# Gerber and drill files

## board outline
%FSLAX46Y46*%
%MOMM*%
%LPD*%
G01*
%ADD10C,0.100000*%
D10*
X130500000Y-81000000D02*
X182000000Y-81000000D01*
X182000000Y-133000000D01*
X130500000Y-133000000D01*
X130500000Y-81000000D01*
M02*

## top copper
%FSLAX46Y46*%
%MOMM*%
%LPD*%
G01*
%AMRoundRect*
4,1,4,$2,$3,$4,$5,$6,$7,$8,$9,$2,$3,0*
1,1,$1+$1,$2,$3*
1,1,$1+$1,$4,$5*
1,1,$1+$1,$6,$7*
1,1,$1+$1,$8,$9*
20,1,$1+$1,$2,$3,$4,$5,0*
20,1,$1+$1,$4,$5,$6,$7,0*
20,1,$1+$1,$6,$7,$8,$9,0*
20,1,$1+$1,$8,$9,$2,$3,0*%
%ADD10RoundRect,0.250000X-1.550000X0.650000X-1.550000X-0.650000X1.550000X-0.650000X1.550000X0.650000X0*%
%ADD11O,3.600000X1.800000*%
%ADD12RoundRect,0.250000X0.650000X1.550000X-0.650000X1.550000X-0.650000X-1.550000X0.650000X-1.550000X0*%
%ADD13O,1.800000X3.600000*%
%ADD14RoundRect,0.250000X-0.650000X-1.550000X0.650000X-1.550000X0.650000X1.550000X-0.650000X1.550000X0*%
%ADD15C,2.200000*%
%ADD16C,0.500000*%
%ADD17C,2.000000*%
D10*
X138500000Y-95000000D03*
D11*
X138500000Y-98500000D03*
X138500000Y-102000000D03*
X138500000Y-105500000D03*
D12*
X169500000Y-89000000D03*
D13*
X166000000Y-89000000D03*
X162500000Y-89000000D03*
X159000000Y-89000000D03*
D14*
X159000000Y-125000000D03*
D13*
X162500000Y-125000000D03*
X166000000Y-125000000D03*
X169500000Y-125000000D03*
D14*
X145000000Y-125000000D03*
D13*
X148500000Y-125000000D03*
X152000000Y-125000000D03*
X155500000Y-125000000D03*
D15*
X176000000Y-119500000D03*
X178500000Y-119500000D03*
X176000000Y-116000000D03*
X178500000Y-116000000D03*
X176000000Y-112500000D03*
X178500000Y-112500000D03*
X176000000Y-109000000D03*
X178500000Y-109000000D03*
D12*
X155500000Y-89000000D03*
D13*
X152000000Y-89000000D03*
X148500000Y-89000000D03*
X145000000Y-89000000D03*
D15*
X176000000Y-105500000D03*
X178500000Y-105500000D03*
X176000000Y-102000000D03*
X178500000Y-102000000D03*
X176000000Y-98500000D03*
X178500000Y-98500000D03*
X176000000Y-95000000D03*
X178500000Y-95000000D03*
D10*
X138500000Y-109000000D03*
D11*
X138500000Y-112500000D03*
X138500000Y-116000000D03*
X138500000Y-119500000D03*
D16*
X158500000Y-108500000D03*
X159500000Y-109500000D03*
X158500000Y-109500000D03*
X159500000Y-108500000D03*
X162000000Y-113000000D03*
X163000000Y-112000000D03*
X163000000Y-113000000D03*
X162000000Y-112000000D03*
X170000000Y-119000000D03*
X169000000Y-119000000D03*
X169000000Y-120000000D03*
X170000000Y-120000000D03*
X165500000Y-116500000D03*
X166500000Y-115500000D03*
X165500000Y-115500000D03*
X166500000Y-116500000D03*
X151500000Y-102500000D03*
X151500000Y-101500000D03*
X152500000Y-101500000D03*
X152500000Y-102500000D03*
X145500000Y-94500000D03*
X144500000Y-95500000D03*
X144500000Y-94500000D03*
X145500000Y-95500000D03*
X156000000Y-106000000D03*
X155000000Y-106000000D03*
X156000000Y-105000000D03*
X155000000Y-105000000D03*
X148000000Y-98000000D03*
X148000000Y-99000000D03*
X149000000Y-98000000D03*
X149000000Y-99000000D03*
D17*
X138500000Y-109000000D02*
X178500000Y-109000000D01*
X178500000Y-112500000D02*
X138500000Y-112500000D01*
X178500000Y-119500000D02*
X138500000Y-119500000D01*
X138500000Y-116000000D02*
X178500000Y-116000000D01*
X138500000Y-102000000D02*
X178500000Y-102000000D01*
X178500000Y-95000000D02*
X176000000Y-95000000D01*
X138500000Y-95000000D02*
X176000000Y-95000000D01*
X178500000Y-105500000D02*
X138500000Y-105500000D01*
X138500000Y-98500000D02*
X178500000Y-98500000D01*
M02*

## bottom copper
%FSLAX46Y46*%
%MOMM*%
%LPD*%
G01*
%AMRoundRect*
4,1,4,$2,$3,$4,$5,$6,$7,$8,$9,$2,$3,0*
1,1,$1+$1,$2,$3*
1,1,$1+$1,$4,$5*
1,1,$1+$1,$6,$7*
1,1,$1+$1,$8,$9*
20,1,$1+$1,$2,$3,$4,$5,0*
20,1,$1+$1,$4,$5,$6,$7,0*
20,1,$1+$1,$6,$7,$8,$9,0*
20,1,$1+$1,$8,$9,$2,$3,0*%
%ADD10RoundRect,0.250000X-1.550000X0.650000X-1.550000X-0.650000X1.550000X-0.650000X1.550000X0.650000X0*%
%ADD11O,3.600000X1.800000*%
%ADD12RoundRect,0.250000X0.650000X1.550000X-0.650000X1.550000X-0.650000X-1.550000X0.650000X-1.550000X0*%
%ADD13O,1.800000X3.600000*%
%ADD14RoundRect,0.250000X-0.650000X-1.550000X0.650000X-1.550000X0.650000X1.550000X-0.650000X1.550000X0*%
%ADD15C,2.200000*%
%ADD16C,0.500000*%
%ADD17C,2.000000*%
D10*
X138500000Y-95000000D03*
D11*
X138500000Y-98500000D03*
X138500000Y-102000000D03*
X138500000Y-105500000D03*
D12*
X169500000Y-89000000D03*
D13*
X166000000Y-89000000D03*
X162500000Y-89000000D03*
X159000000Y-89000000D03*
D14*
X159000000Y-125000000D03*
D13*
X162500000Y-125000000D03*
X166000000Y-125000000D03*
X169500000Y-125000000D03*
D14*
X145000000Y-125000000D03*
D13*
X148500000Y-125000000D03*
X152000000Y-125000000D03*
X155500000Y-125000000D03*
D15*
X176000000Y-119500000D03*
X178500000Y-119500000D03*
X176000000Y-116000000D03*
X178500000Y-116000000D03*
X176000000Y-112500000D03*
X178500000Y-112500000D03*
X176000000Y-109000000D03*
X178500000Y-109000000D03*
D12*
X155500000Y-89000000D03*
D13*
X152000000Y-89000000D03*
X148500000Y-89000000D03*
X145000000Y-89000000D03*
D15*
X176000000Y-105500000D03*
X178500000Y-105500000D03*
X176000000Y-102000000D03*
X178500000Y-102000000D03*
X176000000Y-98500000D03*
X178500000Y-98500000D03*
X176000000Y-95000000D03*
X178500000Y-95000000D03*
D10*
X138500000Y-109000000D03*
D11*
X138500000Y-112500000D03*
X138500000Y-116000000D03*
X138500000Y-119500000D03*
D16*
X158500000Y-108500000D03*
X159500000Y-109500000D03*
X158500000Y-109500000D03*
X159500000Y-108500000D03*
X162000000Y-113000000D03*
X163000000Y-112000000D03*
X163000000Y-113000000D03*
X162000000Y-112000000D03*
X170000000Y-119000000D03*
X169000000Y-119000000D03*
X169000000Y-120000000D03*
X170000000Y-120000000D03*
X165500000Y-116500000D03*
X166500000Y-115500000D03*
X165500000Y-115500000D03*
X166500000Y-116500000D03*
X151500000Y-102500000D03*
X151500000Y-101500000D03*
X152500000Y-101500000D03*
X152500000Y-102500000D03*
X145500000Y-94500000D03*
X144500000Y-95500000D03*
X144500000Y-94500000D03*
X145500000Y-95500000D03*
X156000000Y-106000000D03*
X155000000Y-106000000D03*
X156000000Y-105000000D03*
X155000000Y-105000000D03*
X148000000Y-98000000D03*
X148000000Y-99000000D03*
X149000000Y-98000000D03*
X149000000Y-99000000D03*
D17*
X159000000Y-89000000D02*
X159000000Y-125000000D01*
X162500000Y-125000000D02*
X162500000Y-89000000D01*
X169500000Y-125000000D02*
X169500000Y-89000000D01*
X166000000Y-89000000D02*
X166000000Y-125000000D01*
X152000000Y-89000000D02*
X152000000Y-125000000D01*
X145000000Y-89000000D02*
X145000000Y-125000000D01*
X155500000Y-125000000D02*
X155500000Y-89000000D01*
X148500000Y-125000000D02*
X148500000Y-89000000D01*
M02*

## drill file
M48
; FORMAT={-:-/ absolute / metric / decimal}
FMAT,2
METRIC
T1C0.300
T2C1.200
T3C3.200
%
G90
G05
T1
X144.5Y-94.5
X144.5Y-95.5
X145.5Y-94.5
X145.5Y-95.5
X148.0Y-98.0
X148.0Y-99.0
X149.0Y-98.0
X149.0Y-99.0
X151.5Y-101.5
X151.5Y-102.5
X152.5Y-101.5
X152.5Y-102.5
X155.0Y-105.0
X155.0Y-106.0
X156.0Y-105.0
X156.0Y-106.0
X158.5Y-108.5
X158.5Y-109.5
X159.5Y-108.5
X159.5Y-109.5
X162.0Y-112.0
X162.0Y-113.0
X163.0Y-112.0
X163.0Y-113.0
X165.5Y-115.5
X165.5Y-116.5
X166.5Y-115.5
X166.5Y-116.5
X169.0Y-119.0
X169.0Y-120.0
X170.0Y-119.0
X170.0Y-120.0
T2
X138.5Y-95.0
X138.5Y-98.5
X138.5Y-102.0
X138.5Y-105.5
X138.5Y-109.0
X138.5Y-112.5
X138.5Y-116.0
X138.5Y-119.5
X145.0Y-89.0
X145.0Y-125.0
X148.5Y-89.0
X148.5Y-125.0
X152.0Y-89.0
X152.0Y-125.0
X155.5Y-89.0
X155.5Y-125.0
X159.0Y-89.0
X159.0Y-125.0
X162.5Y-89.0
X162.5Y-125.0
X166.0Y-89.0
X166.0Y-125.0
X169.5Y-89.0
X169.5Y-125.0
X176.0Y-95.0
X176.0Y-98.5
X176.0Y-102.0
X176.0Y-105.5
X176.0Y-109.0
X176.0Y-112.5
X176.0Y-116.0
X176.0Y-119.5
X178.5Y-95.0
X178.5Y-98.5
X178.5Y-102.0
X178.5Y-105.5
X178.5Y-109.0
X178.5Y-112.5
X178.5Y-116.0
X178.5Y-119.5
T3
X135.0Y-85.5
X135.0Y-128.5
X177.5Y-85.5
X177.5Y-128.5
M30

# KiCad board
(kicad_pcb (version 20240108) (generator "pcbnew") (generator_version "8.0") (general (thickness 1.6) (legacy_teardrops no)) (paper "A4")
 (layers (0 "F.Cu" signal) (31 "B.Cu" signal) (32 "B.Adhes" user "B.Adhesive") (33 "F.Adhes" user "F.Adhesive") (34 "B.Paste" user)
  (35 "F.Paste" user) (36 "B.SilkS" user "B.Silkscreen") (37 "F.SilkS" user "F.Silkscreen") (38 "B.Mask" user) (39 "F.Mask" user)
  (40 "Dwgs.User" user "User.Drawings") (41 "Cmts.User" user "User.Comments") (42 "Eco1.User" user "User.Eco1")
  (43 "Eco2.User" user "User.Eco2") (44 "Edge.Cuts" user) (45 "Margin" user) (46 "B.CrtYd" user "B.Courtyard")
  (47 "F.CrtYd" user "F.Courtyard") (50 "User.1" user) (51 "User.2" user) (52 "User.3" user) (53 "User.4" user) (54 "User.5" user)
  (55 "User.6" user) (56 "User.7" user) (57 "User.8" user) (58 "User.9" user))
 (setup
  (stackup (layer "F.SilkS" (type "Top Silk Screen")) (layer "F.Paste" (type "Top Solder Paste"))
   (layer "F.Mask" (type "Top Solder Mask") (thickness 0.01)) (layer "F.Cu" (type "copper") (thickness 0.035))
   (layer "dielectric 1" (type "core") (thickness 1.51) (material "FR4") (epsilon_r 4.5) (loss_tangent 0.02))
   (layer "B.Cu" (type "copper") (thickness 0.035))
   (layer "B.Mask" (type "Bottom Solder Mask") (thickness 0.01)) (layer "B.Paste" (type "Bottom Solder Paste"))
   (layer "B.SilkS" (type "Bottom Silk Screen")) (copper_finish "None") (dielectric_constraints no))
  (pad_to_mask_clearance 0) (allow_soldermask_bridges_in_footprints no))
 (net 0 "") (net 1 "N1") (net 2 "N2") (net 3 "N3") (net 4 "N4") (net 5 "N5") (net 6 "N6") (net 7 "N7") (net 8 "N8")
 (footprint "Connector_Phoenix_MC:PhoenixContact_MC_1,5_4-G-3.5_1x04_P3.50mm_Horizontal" (layer "F.Cu") (at 138.5 95 -90)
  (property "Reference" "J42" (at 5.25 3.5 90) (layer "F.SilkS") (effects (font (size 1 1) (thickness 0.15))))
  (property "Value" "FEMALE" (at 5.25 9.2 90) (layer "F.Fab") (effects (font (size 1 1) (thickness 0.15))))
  (pad "1" thru_hole roundrect (at 0 0 270) (size 1.8 3.6) (drill 1.2) (layers "*.Cu" "*.Mask") (remove_unused_layers no)
   (roundrect_rratio 0.138889) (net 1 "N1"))
  (pad "2" thru_hole oval (at 3.5 0 270) (size 1.8 3.6) (drill 1.2) (layers "*.Cu" "*.Mask") (remove_unused_layers no) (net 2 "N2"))
  (pad "3" thru_hole oval (at 7 0 270) (size 1.8 3.6) (drill 1.2) (layers "*.Cu" "*.Mask") (remove_unused_layers no) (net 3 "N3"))
  (pad "4" thru_hole oval (at 10.5 0 270) (size 1.8 3.6) (drill 1.2) (layers "*.Cu" "*.Mask") (remove_unused_layers no) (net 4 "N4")))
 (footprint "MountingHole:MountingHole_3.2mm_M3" (layer "F.Cu") (at 135 128.5)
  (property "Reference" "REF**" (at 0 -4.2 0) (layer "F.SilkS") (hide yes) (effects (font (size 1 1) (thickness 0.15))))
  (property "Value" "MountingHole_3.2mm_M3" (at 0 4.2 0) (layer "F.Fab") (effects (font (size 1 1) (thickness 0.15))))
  (pad "" np_thru_hole circle (at 0 0) (size 3.2 3.2) (drill 3.2) (layers "F&B.Cu" "*.Mask")))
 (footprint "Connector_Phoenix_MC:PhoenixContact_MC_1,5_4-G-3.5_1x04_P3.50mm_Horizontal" (layer "F.Cu") (at 169.5 89 180)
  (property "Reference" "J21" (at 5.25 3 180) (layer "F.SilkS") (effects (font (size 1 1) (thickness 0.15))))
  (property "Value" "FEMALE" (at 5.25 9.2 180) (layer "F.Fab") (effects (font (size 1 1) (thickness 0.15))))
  (pad "1" thru_hole roundrect (at 0 0 180) (size 1.8 3.6) (drill 1.2) (layers "*.Cu" "*.Mask") (remove_unused_layers no)
   (roundrect_rratio 0.138889) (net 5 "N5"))
  (pad "2" thru_hole oval (at 3.5 0 180) (size 1.8 3.6) (drill 1.2) (layers "*.Cu" "*.Mask") (remove_unused_layers no) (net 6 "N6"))
  (pad "3" thru_hole oval (at 7 0 180) (size 1.8 3.6) (drill 1.2) (layers "*.Cu" "*.Mask") (remove_unused_layers no) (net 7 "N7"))
  (pad "4" thru_hole oval (at 10.5 0 180) (size 1.8 3.6) (drill 1.2) (layers "*.Cu" "*.Mask") (remove_unused_layers no) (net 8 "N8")))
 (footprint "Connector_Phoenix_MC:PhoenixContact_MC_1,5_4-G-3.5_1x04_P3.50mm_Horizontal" (layer "F.Cu") (at 159 125)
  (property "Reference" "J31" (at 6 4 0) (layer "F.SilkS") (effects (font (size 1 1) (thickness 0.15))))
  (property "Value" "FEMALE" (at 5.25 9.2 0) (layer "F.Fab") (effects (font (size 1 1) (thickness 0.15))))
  (pad "1" thru_hole roundrect (at 0 0) (size 1.8 3.6) (drill 1.2) (layers "*.Cu" "*.Mask") (remove_unused_layers no)
   (roundrect_rratio 0.138889) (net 8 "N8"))
  (pad "2" thru_hole oval (at 3.5 0) (size 1.8 3.6) (drill 1.2) (layers "*.Cu" "*.Mask") (remove_unused_layers no) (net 7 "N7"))
  (pad "3" thru_hole oval (at 7 0) (size 1.8 3.6) (drill 1.2) (layers "*.Cu" "*.Mask") (remove_unused_layers no) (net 6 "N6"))
  (pad "4" thru_hole oval (at 10.5 0) (size 1.8 3.6) (drill 1.2) (layers "*.Cu" "*.Mask") (remove_unused_layers no) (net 5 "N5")))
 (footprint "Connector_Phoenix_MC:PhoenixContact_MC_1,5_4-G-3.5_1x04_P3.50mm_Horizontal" (layer "F.Cu") (at 145 125)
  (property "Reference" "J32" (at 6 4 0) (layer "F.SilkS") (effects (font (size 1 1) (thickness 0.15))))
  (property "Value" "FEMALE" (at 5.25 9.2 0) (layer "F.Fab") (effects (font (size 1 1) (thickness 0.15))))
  (pad "1" thru_hole roundrect (at 0 0) (size 1.8 3.6) (drill 1.2) (layers "*.Cu" "*.Mask") (remove_unused_layers no)
   (roundrect_rratio 0.138889) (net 1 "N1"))
  (pad "2" thru_hole oval (at 3.5 0) (size 1.8 3.6) (drill 1.2) (layers "*.Cu" "*.Mask") (remove_unused_layers no) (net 2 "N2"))
  (pad "3" thru_hole oval (at 7 0) (size 1.8 3.6) (drill 1.2) (layers "*.Cu" "*.Mask") (remove_unused_layers no) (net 3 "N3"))
  (pad "4" thru_hole oval (at 10.5 0) (size 1.8 3.6) (drill 1.2) (layers "*.Cu" "*.Mask") (remove_unused_layers no) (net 4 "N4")))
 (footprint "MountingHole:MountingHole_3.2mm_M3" (layer "F.Cu") (at 177.5 85.5)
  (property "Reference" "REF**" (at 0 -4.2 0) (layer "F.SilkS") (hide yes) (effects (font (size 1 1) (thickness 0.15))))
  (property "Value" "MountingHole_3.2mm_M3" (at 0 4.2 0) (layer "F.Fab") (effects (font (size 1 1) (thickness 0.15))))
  (pad "" np_thru_hole circle (at 0 0) (size 3.2 3.2) (drill 3.2) (layers "F&B.Cu" "*.Mask")))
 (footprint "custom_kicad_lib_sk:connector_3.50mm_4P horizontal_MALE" (layer "F.Cu") (at 176 114.25 90)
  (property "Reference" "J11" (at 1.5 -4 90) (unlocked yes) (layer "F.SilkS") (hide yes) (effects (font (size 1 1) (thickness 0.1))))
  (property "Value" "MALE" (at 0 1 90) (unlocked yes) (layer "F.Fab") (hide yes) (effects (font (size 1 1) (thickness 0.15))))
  (pad "1" thru_hole circle (at -5.25 0 90) (size 2.2 2.2) (drill 1.2) (layers "*.Cu" "*.Mask") (remove_unused_layers no) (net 5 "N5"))
  (pad "1" thru_hole circle (at -5.25 2.5 90) (size 2.2 2.2) (drill 1.2) (layers "*.Cu" "*.Mask") (remove_unused_layers no) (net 5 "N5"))
  (pad "2" thru_hole circle (at -1.75 0 90) (size 2.2 2.2) (drill 1.2) (layers "*.Cu" "*.Mask") (remove_unused_layers no) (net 6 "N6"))
  (pad "2" thru_hole circle (at -1.75 2.5 90) (size 2.2 2.2) (drill 1.2) (layers "*.Cu" "*.Mask") (remove_unused_layers no) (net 6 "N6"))
  (pad "3" thru_hole circle (at 1.75 0 90) (size 2.2 2.2) (drill 1.2) (layers "*.Cu" "*.Mask") (remove_unused_layers no) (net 7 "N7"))
  (pad "3" thru_hole circle (at 1.75 2.5 90) (size 2.2 2.2) (drill 1.2) (layers "*.Cu" "*.Mask") (remove_unused_layers no) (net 7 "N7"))
  (pad "4" thru_hole circle (at 5.25 0 90) (size 2.2 2.2) (drill 1.2) (layers "*.Cu" "*.Mask") (remove_unused_layers no) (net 8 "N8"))
  (pad "4" thru_hole circle (at 5.25 2.5 90) (size 2.2 2.2) (drill 1.2) (layers "*.Cu" "*.Mask") (remove_unused_layers no) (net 8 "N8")))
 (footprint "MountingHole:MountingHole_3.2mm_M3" (layer "F.Cu") (at 135 85.5)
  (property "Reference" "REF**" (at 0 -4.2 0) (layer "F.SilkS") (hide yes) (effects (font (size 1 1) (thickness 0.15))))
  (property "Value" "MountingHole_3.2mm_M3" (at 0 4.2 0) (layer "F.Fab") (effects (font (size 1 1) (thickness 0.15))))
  (pad "" np_thru_hole circle (at 0 0) (size 3.2 3.2) (drill 3.2) (layers "F&B.Cu" "*.Mask")))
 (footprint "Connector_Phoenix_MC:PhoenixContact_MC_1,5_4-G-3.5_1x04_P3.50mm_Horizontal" (layer "F.Cu") (at 155.5 89 180)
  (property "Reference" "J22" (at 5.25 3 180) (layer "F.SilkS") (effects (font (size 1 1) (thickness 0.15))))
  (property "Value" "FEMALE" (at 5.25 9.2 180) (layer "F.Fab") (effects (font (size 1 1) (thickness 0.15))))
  (pad "1" thru_hole roundrect (at 0 0 180) (size 1.8 3.6) (drill 1.2) (layers "*.Cu" "*.Mask") (remove_unused_layers no)
   (roundrect_rratio 0.138889) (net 4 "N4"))
  (pad "2" thru_hole oval (at 3.5 0 180) (size 1.8 3.6) (drill 1.2) (layers "*.Cu" "*.Mask") (remove_unused_layers no) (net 3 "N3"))
  (pad "3" thru_hole oval (at 7 0 180) (size 1.8 3.6) (drill 1.2) (layers "*.Cu" "*.Mask") (remove_unused_layers no) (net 2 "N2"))
  (pad "4" thru_hole oval (at 10.5 0 180) (size 1.8 3.6) (drill 1.2) (layers "*.Cu" "*.Mask") (remove_unused_layers no) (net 1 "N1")))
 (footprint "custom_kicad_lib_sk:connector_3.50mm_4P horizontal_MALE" (layer "F.Cu") (at 176 100.25 90)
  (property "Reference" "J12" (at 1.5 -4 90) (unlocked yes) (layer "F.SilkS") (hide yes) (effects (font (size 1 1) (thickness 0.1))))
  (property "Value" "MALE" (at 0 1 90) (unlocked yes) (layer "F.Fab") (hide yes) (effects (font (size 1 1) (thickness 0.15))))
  (pad "1" thru_hole circle (at -5.25 0 90) (size 2.2 2.2) (drill 1.2) (layers "*.Cu" "*.Mask") (remove_unused_layers no) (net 4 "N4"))
  (pad "1" thru_hole circle (at -5.25 2.5 90) (size 2.2 2.2) (drill 1.2) (layers "*.Cu" "*.Mask") (remove_unused_layers no) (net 4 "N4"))
  (pad "2" thru_hole circle (at -1.75 0 90) (size 2.2 2.2) (drill 1.2) (layers "*.Cu" "*.Mask") (remove_unused_layers no) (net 3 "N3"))
  (pad "2" thru_hole circle (at -1.75 2.5 90) (size 2.2 2.2) (drill 1.2) (layers "*.Cu" "*.Mask") (remove_unused_layers no) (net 3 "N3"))
  (pad "3" thru_hole circle (at 1.75 0 90) (size 2.2 2.2) (drill 1.2) (layers "*.Cu" "*.Mask") (remove_unused_layers no) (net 2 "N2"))
  (pad "3" thru_hole circle (at 1.75 2.5 90) (size 2.2 2.2) (drill 1.2) (layers "*.Cu" "*.Mask") (remove_unused_layers no) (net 2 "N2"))
  (pad "4" thru_hole circle (at 5.25 0 90) (size 2.2 2.2) (drill 1.2) (layers "*.Cu" "*.Mask") (remove_unused_layers no) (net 1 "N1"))
  (pad "4" thru_hole circle (at 5.25 2.5 90) (size 2.2 2.2) (drill 1.2) (layers "*.Cu" "*.Mask") (remove_unused_layers no) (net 1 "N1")))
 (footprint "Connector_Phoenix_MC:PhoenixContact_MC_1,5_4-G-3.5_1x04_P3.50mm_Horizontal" (layer "F.Cu") (at 138.5 109 -90)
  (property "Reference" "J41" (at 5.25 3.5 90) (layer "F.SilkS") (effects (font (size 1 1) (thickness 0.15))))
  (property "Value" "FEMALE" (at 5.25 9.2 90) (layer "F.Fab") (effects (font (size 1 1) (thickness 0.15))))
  (pad "1" thru_hole roundrect (at 0 0 270) (size 1.8 3.6) (drill 1.2) (layers "*.Cu" "*.Mask") (remove_unused_layers no)
   (roundrect_rratio 0.138889) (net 8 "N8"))
  (pad "2" thru_hole oval (at 3.5 0 270) (size 1.8 3.6) (drill 1.2) (layers "*.Cu" "*.Mask") (remove_unused_layers no) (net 7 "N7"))
  (pad "3" thru_hole oval (at 7 0 270) (size 1.8 3.6) (drill 1.2) (layers "*.Cu" "*.Mask") (remove_unused_layers no) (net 6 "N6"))
  (pad "4" thru_hole oval (at 10.5 0 270) (size 1.8 3.6) (drill 1.2) (layers "*.Cu" "*.Mask") (remove_unused_layers no) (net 5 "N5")))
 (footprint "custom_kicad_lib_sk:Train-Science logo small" (layer "F.Cu") (at 157.226 107.315 90)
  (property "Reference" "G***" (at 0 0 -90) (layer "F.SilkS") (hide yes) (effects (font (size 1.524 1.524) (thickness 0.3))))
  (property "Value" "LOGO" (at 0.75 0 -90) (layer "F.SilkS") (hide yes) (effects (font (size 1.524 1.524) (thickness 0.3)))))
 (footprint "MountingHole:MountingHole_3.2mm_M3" (layer "F.Cu") (at 177.5 128.5)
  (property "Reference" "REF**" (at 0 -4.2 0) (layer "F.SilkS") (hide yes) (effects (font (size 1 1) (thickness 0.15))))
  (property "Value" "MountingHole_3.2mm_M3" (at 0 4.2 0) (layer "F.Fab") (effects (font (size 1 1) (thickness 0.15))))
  (pad "" np_thru_hole circle (at 0 0) (size 3.2 3.2) (drill 3.2) (layers "*.Cu" "*.Mask")))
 (gr_rect (start 130.5 81) (end 182 133) (stroke (width 0.1) (type default)) (fill none) (layer "Edge.Cuts"))
 (segment (start 138.5 109) (end 178.5 109) (width 2) (layer "F.Cu") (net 8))
 (via (at 158.5 108.5) (size 0.5) (drill 0.3) (layers "F.Cu" "B.Cu") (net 8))
 (via (at 159.5 109.5) (size 0.5) (drill 0.3) (layers "F.Cu" "B.Cu") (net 8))
 (via (at 158.5 109.5) (size 0.5) (drill 0.3) (layers "F.Cu" "B.Cu") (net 8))
 (via (at 159.5 108.5) (size 0.5) (drill 0.3) (layers "F.Cu" "B.Cu") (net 8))
 (segment (start 159 89) (end 159 125) (width 2) (layer "B.Cu") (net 8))
 (segment (start 178.5 112.5) (end 138.5 112.5) (width 2) (layer "F.Cu") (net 7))
 (via (at 162 113) (size 0.5) (drill 0.3) (layers "F.Cu" "B.Cu") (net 7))
 (via (at 163 112) (size 0.5) (drill 0.3) (layers "F.Cu" "B.Cu") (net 7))
 (via (at 163 113) (size 0.5) (drill 0.3) (layers "F.Cu" "B.Cu") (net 7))
 (via (at 162 112) (size 0.5) (drill 0.3) (layers "F.Cu" "B.Cu") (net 7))
 (segment (start 162.5 125) (end 162.5 89) (width 2) (layer "B.Cu") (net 7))
 (segment (start 178.5 119.5) (end 138.5 119.5) (width 2) (layer "F.Cu") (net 5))
 (via (at 170 119) (size 0.5) (drill 0.3) (layers "F.Cu" "B.Cu") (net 5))
 (via (at 169 119) (size 0.5) (drill 0.3) (layers "F.Cu" "B.Cu") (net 5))
 (via (at 169 120) (size 0.5) (drill 0.3) (layers "F.Cu" "B.Cu") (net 5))
 (via (at 170 120) (size 0.5) (drill 0.3) (layers "F.Cu" "B.Cu") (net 5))
 (segment (start 169.5 125) (end 169.5 89) (width 2) (layer "B.Cu") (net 5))
 (segment (start 138.5 116) (end 178.5 116) (width 2) (layer "F.Cu") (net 6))
 (via (at 165.5 116.5) (size 0.5) (drill 0.3) (layers "F.Cu" "B.Cu") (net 6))
 (via (at 166.5 115.5) (size 0.5) (drill 0.3) (layers "F.Cu" "B.Cu") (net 6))
 (via (at 165.5 115.5) (size 0.5) (drill 0.3) (layers "F.Cu" "B.Cu") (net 6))
 (via (at 166.5 116.5) (size 0.5) (drill 0.3) (layers "F.Cu" "B.Cu") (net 6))
 (segment (start 166 89) (end 166 125) (width 2) (layer "B.Cu") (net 6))
 (segment (start 138.5 102) (end 178.5 102) (width 2) (layer "F.Cu") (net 3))
 (via (at 151.5 102.5) (size 0.5) (drill 0.3) (layers "F.Cu" "B.Cu") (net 3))
 (via (at 151.5 101.5) (size 0.5) (drill 0.3) (layers "F.Cu" "B.Cu") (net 3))
 (via (at 152.5 101.5) (size 0.5) (drill 0.3) (layers "F.Cu" "B.Cu") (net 3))
 (via (at 152.5 102.5) (size 0.5) (drill 0.3) (layers "F.Cu" "B.Cu") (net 3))
 (segment (start 152 89) (end 152 125) (width 2) (layer "B.Cu") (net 3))
 (segment (start 178.5 95) (end 176 95) (width 2) (layer "F.Cu") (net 1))
 (segment (start 138.5 95) (end 176 95) (width 2) (layer "F.Cu") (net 1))
 (via (at 145.5 94.5) (size 0.5) (drill 0.3) (layers "F.Cu" "B.Cu") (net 1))
 (via (at 144.5 95.5) (size 0.5) (drill 0.3) (layers "F.Cu" "B.Cu") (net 1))
 (via (at 144.5 94.5) (size 0.5) (drill 0.3) (layers "F.Cu" "B.Cu") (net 1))
 (via (at 145.5 95.5) (size 0.5) (drill 0.3) (layers "F.Cu" "B.Cu") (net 1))
 (segment (start 145 89) (end 145 125) (width 2) (layer "B.Cu") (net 1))
 (segment (start 178.5 105.5) (end 138.5 105.5) (width 2) (layer "F.Cu") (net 4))
 (via (at 156 106) (size 0.5) (drill 0.3) (layers "F.Cu" "B.Cu") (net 4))
 (via (at 155 106) (size 0.5) (drill 0.3) (layers "F.Cu" "B.Cu") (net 4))
 (via (at 156 105) (size 0.5) (drill 0.3) (layers "F.Cu" "B.Cu") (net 4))
 (via (at 155 105) (size 0.5) (drill 0.3) (layers "F.Cu" "B.Cu") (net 4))
 (segment (start 155.5 125) (end 155.5 89) (width 2) (layer "B.Cu") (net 4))
 (segment (start 138.5 98.5) (end 178.5 98.5) (width 2) (layer "F.Cu") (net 2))
 (via (at 148 98) (size 0.5) (drill 0.3) (layers "F.Cu" "B.Cu") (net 2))
 (via (at 148 99) (size 0.5) (drill 0.3) (layers "F.Cu" "B.Cu") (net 2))
 (via (at 149 98) (size 0.5) (drill 0.3) (layers "F.Cu" "B.Cu") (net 2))
 (via (at 149 99) (size 0.5) (drill 0.3) (layers "F.Cu" "B.Cu") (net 2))
 (segment (start 148.5 125) (end 148.5 89) (width 2) (layer "B.Cu") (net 2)))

